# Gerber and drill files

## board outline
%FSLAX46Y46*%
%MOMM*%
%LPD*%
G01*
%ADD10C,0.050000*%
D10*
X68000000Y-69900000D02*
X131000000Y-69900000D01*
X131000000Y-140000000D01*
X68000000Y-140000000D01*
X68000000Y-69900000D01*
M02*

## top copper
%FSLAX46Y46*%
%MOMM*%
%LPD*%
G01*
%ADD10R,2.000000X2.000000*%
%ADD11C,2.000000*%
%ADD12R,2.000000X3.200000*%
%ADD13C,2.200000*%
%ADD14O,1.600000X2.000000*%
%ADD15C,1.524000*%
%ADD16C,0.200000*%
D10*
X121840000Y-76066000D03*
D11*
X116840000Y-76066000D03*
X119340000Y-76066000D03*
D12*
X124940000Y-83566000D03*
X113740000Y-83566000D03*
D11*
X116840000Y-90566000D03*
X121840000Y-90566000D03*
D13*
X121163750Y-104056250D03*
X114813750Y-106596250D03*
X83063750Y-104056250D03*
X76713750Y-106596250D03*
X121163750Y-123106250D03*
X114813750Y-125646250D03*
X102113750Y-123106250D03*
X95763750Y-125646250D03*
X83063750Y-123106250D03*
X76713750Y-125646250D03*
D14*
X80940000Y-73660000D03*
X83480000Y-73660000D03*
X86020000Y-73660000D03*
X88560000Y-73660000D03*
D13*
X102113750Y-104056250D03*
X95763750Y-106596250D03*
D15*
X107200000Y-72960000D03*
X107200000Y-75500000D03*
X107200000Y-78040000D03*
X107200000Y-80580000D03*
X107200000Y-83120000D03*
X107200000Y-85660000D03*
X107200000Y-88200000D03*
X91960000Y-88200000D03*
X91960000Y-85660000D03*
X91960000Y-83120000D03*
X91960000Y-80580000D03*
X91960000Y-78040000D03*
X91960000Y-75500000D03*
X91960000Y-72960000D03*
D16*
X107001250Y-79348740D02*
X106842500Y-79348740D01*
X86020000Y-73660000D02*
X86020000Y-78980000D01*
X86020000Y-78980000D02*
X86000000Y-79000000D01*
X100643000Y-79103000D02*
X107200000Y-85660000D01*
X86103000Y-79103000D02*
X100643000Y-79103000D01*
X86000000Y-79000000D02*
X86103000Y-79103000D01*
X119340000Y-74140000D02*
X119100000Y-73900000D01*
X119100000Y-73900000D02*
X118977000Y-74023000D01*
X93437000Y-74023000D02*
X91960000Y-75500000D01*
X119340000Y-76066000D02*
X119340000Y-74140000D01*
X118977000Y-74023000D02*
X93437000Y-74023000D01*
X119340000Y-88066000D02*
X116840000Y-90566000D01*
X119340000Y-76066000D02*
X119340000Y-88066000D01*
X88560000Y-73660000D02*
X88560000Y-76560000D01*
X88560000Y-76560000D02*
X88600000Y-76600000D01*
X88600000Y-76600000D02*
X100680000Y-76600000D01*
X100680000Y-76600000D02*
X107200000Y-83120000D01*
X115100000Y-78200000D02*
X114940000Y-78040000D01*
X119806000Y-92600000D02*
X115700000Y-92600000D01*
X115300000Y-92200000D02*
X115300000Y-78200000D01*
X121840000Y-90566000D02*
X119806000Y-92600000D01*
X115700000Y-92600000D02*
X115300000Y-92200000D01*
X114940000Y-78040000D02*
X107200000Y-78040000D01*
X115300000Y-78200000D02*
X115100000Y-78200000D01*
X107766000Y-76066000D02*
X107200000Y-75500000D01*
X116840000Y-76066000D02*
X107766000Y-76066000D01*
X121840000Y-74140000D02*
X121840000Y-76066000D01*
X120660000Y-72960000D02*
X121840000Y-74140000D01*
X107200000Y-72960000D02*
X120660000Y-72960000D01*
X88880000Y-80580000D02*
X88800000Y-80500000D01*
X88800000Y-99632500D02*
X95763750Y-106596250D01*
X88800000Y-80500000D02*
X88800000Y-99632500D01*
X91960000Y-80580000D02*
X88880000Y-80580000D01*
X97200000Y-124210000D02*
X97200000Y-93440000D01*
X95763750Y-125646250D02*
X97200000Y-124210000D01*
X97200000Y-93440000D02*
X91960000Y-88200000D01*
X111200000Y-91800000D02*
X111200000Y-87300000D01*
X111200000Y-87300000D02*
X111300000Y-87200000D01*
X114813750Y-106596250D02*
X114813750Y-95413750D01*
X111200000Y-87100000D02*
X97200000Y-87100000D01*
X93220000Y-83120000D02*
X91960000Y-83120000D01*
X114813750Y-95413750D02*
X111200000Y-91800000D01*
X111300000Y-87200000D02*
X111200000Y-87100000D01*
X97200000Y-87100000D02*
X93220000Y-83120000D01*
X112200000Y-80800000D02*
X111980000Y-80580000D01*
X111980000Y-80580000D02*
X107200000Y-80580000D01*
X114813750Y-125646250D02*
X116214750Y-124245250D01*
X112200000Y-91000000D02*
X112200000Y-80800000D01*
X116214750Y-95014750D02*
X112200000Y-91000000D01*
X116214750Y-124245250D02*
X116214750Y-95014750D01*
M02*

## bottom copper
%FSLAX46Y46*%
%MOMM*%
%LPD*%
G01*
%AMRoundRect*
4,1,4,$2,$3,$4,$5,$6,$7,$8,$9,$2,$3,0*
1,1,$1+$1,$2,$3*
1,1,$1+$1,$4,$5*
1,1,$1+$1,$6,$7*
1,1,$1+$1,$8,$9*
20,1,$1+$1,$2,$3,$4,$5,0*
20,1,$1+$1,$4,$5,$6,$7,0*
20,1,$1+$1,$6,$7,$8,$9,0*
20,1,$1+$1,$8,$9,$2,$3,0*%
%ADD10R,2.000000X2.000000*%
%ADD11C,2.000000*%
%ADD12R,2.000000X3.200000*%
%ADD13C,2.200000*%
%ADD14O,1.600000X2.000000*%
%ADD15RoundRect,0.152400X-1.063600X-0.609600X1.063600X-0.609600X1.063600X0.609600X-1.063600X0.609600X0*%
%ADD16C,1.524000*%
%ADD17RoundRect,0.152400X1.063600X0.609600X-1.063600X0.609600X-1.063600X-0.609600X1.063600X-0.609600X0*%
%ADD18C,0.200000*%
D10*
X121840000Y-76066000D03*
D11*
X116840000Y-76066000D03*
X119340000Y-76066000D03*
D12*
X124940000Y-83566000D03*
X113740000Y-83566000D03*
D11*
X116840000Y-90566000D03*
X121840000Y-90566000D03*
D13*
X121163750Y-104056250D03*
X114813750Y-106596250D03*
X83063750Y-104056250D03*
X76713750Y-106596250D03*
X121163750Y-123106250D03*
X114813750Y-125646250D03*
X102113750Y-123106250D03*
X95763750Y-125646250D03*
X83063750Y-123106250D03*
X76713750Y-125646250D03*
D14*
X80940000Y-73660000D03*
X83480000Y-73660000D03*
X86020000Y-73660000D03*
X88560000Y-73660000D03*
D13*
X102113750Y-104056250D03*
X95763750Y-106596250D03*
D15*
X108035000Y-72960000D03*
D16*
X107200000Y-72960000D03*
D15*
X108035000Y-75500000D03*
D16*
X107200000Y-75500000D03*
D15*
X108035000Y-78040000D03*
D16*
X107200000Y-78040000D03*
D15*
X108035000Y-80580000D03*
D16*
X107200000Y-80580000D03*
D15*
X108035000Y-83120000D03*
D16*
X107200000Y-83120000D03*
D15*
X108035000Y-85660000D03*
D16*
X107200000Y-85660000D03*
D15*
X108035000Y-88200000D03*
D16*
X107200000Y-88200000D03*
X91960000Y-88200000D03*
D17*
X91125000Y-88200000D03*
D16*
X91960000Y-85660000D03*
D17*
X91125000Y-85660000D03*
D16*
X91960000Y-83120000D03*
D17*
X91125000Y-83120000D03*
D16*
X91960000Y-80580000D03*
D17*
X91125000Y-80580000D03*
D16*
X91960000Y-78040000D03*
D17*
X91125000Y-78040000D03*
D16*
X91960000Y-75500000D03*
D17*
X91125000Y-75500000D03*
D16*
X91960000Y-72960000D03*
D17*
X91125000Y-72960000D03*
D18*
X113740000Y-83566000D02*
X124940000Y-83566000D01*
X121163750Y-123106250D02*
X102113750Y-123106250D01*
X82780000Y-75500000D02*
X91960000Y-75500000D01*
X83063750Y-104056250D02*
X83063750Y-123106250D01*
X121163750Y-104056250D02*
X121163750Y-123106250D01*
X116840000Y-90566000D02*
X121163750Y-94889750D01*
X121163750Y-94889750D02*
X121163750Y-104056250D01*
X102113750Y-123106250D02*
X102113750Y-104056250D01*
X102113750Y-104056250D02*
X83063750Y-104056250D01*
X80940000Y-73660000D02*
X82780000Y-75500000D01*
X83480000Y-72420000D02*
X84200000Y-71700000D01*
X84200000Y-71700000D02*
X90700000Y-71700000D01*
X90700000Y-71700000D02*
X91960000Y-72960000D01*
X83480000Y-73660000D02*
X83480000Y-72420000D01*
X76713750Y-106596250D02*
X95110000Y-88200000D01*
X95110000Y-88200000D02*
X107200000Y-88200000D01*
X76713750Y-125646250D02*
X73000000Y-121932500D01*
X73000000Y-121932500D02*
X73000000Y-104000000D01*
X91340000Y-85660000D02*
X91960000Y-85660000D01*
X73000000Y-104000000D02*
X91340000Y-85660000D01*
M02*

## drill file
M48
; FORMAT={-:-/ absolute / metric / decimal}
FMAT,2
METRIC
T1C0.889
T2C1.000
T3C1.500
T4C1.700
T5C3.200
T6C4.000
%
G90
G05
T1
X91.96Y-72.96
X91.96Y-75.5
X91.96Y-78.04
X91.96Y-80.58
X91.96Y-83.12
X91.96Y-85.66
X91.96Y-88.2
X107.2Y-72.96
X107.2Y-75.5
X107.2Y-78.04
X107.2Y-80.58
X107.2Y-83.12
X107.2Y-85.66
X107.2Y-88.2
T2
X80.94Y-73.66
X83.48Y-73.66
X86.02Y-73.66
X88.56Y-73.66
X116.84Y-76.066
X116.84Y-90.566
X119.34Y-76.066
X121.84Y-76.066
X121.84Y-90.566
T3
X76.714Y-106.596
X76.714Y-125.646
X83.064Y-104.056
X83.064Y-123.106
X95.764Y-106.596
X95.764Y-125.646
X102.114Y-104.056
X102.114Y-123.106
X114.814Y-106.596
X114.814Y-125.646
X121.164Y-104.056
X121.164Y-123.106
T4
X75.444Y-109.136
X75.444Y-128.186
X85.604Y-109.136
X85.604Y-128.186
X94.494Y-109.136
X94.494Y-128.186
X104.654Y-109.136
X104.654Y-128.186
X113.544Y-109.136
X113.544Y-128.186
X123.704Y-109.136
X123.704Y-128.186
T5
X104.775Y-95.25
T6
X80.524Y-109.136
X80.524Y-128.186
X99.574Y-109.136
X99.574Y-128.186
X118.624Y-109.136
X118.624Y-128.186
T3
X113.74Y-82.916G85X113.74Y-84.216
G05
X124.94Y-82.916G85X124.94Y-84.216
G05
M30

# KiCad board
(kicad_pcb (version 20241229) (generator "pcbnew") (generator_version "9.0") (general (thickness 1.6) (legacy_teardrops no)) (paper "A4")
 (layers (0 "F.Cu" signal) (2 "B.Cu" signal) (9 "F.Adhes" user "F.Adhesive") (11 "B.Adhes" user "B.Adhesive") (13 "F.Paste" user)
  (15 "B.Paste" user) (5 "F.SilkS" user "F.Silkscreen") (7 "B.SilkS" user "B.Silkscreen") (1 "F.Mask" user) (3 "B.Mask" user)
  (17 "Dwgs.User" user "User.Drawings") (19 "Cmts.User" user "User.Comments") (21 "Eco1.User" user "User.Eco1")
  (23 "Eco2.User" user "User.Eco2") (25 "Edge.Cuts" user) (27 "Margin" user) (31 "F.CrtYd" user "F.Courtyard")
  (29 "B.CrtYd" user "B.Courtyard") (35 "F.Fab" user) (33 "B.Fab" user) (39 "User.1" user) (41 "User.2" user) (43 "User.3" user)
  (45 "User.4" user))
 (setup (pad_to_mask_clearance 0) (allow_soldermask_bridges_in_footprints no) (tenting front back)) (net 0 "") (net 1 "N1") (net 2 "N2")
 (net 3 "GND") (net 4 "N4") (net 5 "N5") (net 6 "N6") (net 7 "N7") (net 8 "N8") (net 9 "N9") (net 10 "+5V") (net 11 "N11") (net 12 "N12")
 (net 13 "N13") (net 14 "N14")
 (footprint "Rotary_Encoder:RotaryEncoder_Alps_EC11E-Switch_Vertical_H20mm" (layer "F.Cu") (at 121.84 76.066 -90)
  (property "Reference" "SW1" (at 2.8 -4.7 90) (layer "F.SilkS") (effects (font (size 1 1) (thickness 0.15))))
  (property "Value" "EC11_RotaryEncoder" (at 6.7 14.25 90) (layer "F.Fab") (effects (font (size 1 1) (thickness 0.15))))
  (pad "A" thru_hole rect (at 0 0 270) (size 2 2) (drill 1) (layers "*.Cu" "*.Mask") (remove_unused_layers no) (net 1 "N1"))
  (pad "B" thru_hole circle (at 0 5 270) (size 2 2) (drill 1) (layers "*.Cu" "*.Mask") (remove_unused_layers no) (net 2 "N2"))
  (pad "C" thru_hole circle (at 0 2.5 270) (size 2 2) (drill 1) (layers "*.Cu" "*.Mask") (remove_unused_layers no) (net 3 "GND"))
  (pad "MP" thru_hole rect (at 7.5 -3.1 270) (size 3.2 2) (drill oval 2.8 1.5) (layers "*.Cu" "*.Mask") (remove_unused_layers no))
  (pad "MP" thru_hole rect (at 7.5 8.1 270) (size 3.2 2) (drill oval 2.8 1.5) (layers "*.Cu" "*.Mask") (remove_unused_layers no))
  (pad "S1" thru_hole circle (at 14.5 5 270) (size 2 2) (drill 1) (layers "*.Cu" "*.Mask") (remove_unused_layers no) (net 3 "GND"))
  (pad "S2" thru_hole circle (at 14.5 0 270) (size 2 2) (drill 1) (layers "*.Cu" "*.Mask") (remove_unused_layers no) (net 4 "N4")))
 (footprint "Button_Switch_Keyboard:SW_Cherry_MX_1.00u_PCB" (layer "F.Cu") (at 121.16375 104.05625)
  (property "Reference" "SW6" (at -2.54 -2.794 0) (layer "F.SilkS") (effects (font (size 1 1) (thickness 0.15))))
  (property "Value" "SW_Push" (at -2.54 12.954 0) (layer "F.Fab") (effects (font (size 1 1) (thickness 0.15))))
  (pad "" np_thru_hole circle (at -7.62 5.08) (size 1.7 1.7) (drill 1.7) (layers "*.Cu" "*.Mask"))
  (pad "" np_thru_hole circle (at -2.54 5.08) (size 4 4) (drill 4) (layers "*.Cu" "*.Mask"))
  (pad "" np_thru_hole circle (at 2.54 5.08) (size 1.7 1.7) (drill 1.7) (layers "*.Cu" "*.Mask"))
  (pad "1" thru_hole circle (at 0 0) (size 2.2 2.2) (drill 1.5) (layers "*.Cu" "*.Mask") (remove_unused_layers no) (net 3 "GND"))
  (pad "2" thru_hole circle (at -6.35 2.54) (size 2.2 2.2) (drill 1.5) (layers "*.Cu" "*.Mask") (remove_unused_layers no) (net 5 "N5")))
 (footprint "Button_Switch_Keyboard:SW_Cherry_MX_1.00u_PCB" (layer "F.Cu") (at 83.06375 104.05625)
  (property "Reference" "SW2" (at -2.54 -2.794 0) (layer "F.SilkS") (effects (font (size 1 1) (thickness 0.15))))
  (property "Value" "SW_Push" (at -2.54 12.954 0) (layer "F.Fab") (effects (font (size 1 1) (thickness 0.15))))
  (pad "" np_thru_hole circle (at -7.62 5.08) (size 1.7 1.7) (drill 1.7) (layers "*.Cu" "*.Mask"))
  (pad "" np_thru_hole circle (at -2.54 5.08) (size 4 4) (drill 4) (layers "*.Cu" "*.Mask"))
  (pad "" np_thru_hole circle (at 2.54 5.08) (size 1.7 1.7) (drill 1.7) (layers "*.Cu" "*.Mask"))
  (pad "1" thru_hole circle (at 0 0) (size 2.2 2.2) (drill 1.5) (layers "*.Cu" "*.Mask") (remove_unused_layers no) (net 3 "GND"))
  (pad "2" thru_hole circle (at -6.35 2.54) (size 2.2 2.2) (drill 1.5) (layers "*.Cu" "*.Mask") (remove_unused_layers no) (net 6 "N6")))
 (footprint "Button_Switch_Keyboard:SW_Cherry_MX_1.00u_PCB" (layer "F.Cu") (at 121.16375 123.10625)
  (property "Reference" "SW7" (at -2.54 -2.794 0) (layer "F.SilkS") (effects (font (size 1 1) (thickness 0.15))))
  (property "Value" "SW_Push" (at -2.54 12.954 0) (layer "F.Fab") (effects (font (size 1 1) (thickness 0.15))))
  (pad "" np_thru_hole circle (at -7.62 5.08) (size 1.7 1.7) (drill 1.7) (layers "*.Cu" "*.Mask"))
  (pad "" np_thru_hole circle (at -2.54 5.08) (size 4 4) (drill 4) (layers "*.Cu" "*.Mask"))
  (pad "" np_thru_hole circle (at 2.54 5.08) (size 1.7 1.7) (drill 1.7) (layers "*.Cu" "*.Mask"))
  (pad "1" thru_hole circle (at 0 0) (size 2.2 2.2) (drill 1.5) (layers "*.Cu" "*.Mask") (remove_unused_layers no) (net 3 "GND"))
  (pad "2" thru_hole circle (at -6.35 2.54) (size 2.2 2.2) (drill 1.5) (layers "*.Cu" "*.Mask") (remove_unused_layers no) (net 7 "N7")))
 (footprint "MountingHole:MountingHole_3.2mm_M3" (layer "F.Cu") (at 104.775 95.25)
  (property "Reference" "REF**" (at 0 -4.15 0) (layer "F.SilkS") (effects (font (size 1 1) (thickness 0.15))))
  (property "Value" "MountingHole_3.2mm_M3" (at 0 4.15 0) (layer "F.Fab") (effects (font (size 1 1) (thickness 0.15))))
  (pad "" np_thru_hole circle (at 0 0) (size 3.2 3.2) (drill 3.2) (layers "*.Cu" "*.Mask")))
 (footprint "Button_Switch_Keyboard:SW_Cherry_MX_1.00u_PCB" (layer "F.Cu") (at 102.11375 123.10625)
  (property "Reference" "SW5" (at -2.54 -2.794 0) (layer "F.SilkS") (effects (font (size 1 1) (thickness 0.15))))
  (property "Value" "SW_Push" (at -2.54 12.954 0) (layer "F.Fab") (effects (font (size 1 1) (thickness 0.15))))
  (pad "" np_thru_hole circle (at -7.62 5.08) (size 1.7 1.7) (drill 1.7) (layers "*.Cu" "*.Mask"))
  (pad "" np_thru_hole circle (at -2.54 5.08) (size 4 4) (drill 4) (layers "*.Cu" "*.Mask"))
  (pad "" np_thru_hole circle (at 2.54 5.08) (size 1.7 1.7) (drill 1.7) (layers "*.Cu" "*.Mask"))
  (pad "1" thru_hole circle (at 0 0) (size 2.2 2.2) (drill 1.5) (layers "*.Cu" "*.Mask") (remove_unused_layers no) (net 3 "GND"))
  (pad "2" thru_hole circle (at -6.35 2.54) (size 2.2 2.2) (drill 1.5) (layers "*.Cu" "*.Mask") (remove_unused_layers no) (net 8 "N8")))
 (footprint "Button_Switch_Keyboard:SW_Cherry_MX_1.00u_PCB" (layer "F.Cu") (at 83.06375 123.10625)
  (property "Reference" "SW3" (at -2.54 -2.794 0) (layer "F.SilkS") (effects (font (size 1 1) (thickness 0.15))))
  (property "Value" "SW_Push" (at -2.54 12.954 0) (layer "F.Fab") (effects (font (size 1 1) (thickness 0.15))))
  (pad "" np_thru_hole circle (at -7.62 5.08) (size 1.7 1.7) (drill 1.7) (layers "*.Cu" "*.Mask"))
  (pad "" np_thru_hole circle (at -2.54 5.08) (size 4 4) (drill 4) (layers "*.Cu" "*.Mask"))
  (pad "" np_thru_hole circle (at 2.54 5.08) (size 1.7 1.7) (drill 1.7) (layers "*.Cu" "*.Mask"))
  (pad "1" thru_hole circle (at 0 0) (size 2.2 2.2) (drill 1.5) (layers "*.Cu" "*.Mask") (remove_unused_layers no) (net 3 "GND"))
  (pad "2" thru_hole circle (at -6.35 2.54) (size 2.2 2.2) (drill 1.5) (layers "*.Cu" "*.Mask") (remove_unused_layers no) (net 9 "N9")))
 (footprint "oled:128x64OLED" (layer "F.Cu") (at 84.56 84.26)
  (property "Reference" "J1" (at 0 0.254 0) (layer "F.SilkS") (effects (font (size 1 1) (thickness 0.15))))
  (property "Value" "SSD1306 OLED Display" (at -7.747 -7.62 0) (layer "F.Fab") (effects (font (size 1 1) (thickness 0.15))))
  (pad "1" thru_hole oval (at -3.62 -10.6 90) (size 2 1.6) (drill 1) (layers "*.Cu" "*.Mask") (remove_unused_layers no) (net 3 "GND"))
  (pad "2" thru_hole oval (at -1.08 -10.6 90) (size 2 1.6) (drill 1) (layers "*.Cu" "*.Mask") (remove_unused_layers no) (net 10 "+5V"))
  (pad "3" thru_hole oval (at 1.46 -10.6 90) (size 2 1.6) (drill 1) (layers "*.Cu" "*.Mask") (remove_unused_layers no) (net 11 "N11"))
  (pad "4" thru_hole oval (at 4 -10.6 90) (size 2 1.6) (drill 1) (layers "*.Cu" "*.Mask") (remove_unused_layers no) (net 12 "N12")))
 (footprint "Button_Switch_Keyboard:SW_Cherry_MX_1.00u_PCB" (layer "F.Cu") (at 102.11375 104.05625)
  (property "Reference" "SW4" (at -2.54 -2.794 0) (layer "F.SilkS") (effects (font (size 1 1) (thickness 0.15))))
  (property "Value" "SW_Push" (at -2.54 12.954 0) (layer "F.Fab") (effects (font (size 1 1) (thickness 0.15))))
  (pad "" np_thru_hole circle (at -7.62 5.08) (size 1.7 1.7) (drill 1.7) (layers "*.Cu" "*.Mask"))
  (pad "" np_thru_hole circle (at -2.54 5.08) (size 4 4) (drill 4) (layers "*.Cu" "*.Mask"))
  (pad "" np_thru_hole circle (at 2.54 5.08) (size 1.7 1.7) (drill 1.7) (layers "*.Cu" "*.Mask"))
  (pad "1" thru_hole circle (at 0 0) (size 2.2 2.2) (drill 1.5) (layers "*.Cu" "*.Mask") (remove_unused_layers no) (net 3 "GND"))
  (pad "2" thru_hole circle (at -6.35 2.54) (size 2.2 2.2) (drill 1.5) (layers "*.Cu" "*.Mask") (remove_unused_layers no) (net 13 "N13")))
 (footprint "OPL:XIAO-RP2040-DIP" (layer "B.Cu") (at 99.58 80.58 180)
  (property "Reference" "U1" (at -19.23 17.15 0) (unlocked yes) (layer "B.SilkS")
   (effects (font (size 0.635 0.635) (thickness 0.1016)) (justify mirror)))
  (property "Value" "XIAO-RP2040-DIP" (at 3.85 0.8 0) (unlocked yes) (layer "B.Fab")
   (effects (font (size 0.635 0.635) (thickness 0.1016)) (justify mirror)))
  (pad "1" smd roundrect (at -8.455 7.62) (size 2.432 1.524) (layers "B.Cu" "B.Mask") (roundrect_rratio 0.1) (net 1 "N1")
   (thermal_bridge_angle 45))
  (pad "1" thru_hole circle (at -7.62 7.62) (size 1.524 1.524) (drill 0.889) (layers "*.Cu" "*.Mask") (remove_unused_layers no) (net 1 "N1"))
  (pad "2" smd roundrect (at -8.455 5.08) (size 2.432 1.524) (layers "B.Cu" "B.Mask") (roundrect_rratio 0.1) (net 2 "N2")
   (thermal_bridge_angle 45))
  (pad "2" thru_hole circle (at -7.62 5.08) (size 1.524 1.524) (drill 0.889) (layers "*.Cu" "*.Mask") (remove_unused_layers no) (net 2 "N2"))
  (pad "3" smd roundrect (at -8.455 2.54) (size 2.432 1.524) (layers "B.Cu" "B.Mask") (roundrect_rratio 0.1) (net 4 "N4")
   (thermal_bridge_angle 45))
  (pad "3" thru_hole circle (at -7.62 2.54) (size 1.524 1.524) (drill 0.889) (layers "*.Cu" "*.Mask") (remove_unused_layers no) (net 4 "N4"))
  (pad "4" smd roundrect (at -8.455 0) (size 2.432 1.524) (layers "B.Cu" "B.Mask") (roundrect_rratio 0.1) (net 7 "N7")
   (thermal_bridge_angle 45))
  (pad "4" thru_hole circle (at -7.62 0) (size 1.524 1.524) (drill 0.889) (layers "*.Cu" "*.Mask") (remove_unused_layers no) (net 7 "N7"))
  (pad "5" smd roundrect (at -8.455 -2.54) (size 2.432 1.524) (layers "B.Cu" "B.Mask") (roundrect_rratio 0.1) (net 12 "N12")
   (thermal_bridge_angle 45))
  (pad "5" thru_hole circle (at -7.62 -2.54) (size 1.524 1.524) (drill 0.889) (layers "*.Cu" "*.Mask") (remove_unused_layers no)
   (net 12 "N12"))
  (pad "6" smd roundrect (at -8.455 -5.08) (size 2.432 1.524) (layers "B.Cu" "B.Mask") (roundrect_rratio 0.1) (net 11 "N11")
   (thermal_bridge_angle 45))
  (pad "6" thru_hole circle (at -7.62 -5.08) (size 1.524 1.524) (drill 0.889) (layers "*.Cu" "*.Mask") (remove_unused_layers no)
   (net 11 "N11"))
  (pad "7" smd roundrect (at -8.455 -7.62) (size 2.432 1.524) (layers "B.Cu" "B.Mask") (roundrect_rratio 0.1) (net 6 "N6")
   (thermal_bridge_angle 45))
  (pad "7" thru_hole circle (at -7.62 -7.62) (size 1.524 1.524) (drill 0.889) (layers "*.Cu" "*.Mask") (remove_unused_layers no)
   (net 6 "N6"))
  (pad "8" thru_hole circle (at 7.62 -7.62 180) (size 1.524 1.524) (drill 0.889) (layers "*.Cu" "*.Mask") (remove_unused_layers no)
   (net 8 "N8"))
  (pad "8" smd roundrect (at 8.455 -7.62 180) (size 2.432 1.524) (layers "B.Cu" "B.Mask") (roundrect_rratio 0.1) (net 8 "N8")
   (thermal_bridge_angle 45))
  (pad "9" thru_hole circle (at 7.62 -5.08 180) (size 1.524 1.524) (drill 0.889) (layers "*.Cu" "*.Mask") (remove_unused_layers no)
   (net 9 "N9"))
  (pad "9" smd roundrect (at 8.455 -5.08 180) (size 2.432 1.524) (layers "B.Cu" "B.Mask") (roundrect_rratio 0.1) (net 9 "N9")
   (thermal_bridge_angle 45))
  (pad "10" thru_hole circle (at 7.62 -2.54 180) (size 1.524 1.524) (drill 0.889) (layers "*.Cu" "*.Mask") (remove_unused_layers no)
   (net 5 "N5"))
  (pad "10" smd roundrect (at 8.455 -2.54 180) (size 2.432 1.524) (layers "B.Cu" "B.Mask") (roundrect_rratio 0.1) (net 5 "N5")
   (thermal_bridge_angle 45))
  (pad "11" thru_hole circle (at 7.62 0 180) (size 1.524 1.524) (drill 0.889) (layers "*.Cu" "*.Mask") (remove_unused_layers no)
   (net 13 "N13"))
  (pad "11" smd roundrect (at 8.455 0 180) (size 2.432 1.524) (layers "B.Cu" "B.Mask") (roundrect_rratio 0.1) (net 13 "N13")
   (thermal_bridge_angle 45))
  (pad "12" thru_hole circle (at 7.62 2.54 180) (size 1.524 1.524) (drill 0.889) (layers "*.Cu" "*.Mask") (remove_unused_layers no)
   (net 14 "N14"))
  (pad "12" smd roundrect (at 8.455 2.54 180) (size 2.432 1.524) (layers "B.Cu" "B.Mask") (roundrect_rratio 0.1) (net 14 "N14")
   (thermal_bridge_angle 45))
  (pad "13" thru_hole circle (at 7.62 5.08 180) (size 1.524 1.524) (drill 0.889) (layers "*.Cu" "*.Mask") (remove_unused_layers no)
   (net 3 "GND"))
  (pad "13" smd roundrect (at 8.455 5.08 180) (size 2.432 1.524) (layers "B.Cu" "B.Mask") (roundrect_rratio 0.1) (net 3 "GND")
   (thermal_bridge_angle 45))
  (pad "14" thru_hole circle (at 7.62 7.62 180) (size 1.524 1.524) (drill 0.889) (layers "*.Cu" "*.Mask") (remove_unused_layers no)
   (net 10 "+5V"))
  (pad "14" smd roundrect (at 8.455 7.62 180) (size 2.432 1.524) (layers "B.Cu" "B.Mask") (roundrect_rratio 0.1) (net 10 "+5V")
   (thermal_bridge_angle 45)))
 (gr_rect (start 68 69.9) (end 131 140) (stroke (width 0.05) (type default)) (fill no) (layer "Edge.Cuts"))
 (segment (start 107.00125 79.34874) (end 106.8425 79.34874) (width 0.2) (layer "F.Cu") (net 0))
 (segment (start 113.74 83.566) (end 124.94 83.566) (width 0.2) (layer "B.Cu") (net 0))
 (segment (start 86.02 73.66) (end 86.02 78.98) (width 0.2) (layer "F.Cu") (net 11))
 (segment (start 86.02 78.98) (end 86 79) (width 0.2) (layer "F.Cu") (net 11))
 (segment (start 100.643 79.103) (end 107.2 85.66) (width 0.2) (layer "F.Cu") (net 11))
 (segment (start 86.103 79.103) (end 100.643 79.103) (width 0.2) (layer "F.Cu") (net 11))
 (segment (start 86 79) (end 86.103 79.103) (width 0.2) (layer "F.Cu") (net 11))
 (segment (start 119.34 74.14) (end 119.1 73.9) (width 0.2) (layer "F.Cu") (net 3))
 (segment (start 119.1 73.9) (end 118.977 74.023) (width 0.2) (layer "F.Cu") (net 3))
 (segment (start 93.437 74.023) (end 91.96 75.5) (width 0.2) (layer "F.Cu") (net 3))
 (segment (start 119.34 76.066) (end 119.34 74.14) (width 0.2) (layer "F.Cu") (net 3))
 (segment (start 118.977 74.023) (end 93.437 74.023) (width 0.2) (layer "F.Cu") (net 3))
 (segment (start 119.34 88.066) (end 116.84 90.566) (width 0.2) (layer "F.Cu") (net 3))
 (segment (start 119.34 76.066) (end 119.34 88.066) (width 0.2) (layer "F.Cu") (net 3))
 (segment (start 121.16375 123.10625) (end 102.11375 123.10625) (width 0.2) (layer "B.Cu") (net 3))
 (segment (start 82.78 75.5) (end 91.96 75.5) (width 0.2) (layer "B.Cu") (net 3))
 (segment (start 83.06375 104.05625) (end 83.06375 123.10625) (width 0.2) (layer "B.Cu") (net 3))
 (segment (start 121.16375 104.05625) (end 121.16375 123.10625) (width 0.2) (layer "B.Cu") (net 3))
 (segment (start 116.84 90.566) (end 121.16375 94.88975) (width 0.2) (layer "B.Cu") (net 3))
 (segment (start 121.16375 94.88975) (end 121.16375 104.05625) (width 0.2) (layer "B.Cu") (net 3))
 (segment (start 102.11375 123.10625) (end 102.11375 104.05625) (width 0.2) (layer "B.Cu") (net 3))
 (segment (start 102.11375 104.05625) (end 83.06375 104.05625) (width 0.2) (layer "B.Cu") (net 3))
 (segment (start 80.94 73.66) (end 82.78 75.5) (width 0.2) (layer "B.Cu") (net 3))
 (segment (start 88.56 73.66) (end 88.56 76.56) (width 0.2) (layer "F.Cu") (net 12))
 (segment (start 88.56 76.56) (end 88.6 76.6) (width 0.2) (layer "F.Cu") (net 12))
 (segment (start 88.6 76.6) (end 100.68 76.6) (width 0.2) (layer "F.Cu") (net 12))
 (segment (start 100.68 76.6) (end 107.2 83.12) (width 0.2) (layer "F.Cu") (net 12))
 (segment (start 83.48 72.42) (end 84.2 71.7) (width 0.2) (layer "B.Cu") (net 10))
 (segment (start 84.2 71.7) (end 90.7 71.7) (width 0.2) (layer "B.Cu") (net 10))
 (segment (start 90.7 71.7) (end 91.96 72.96) (width 0.2) (layer "B.Cu") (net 10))
 (segment (start 83.48 73.66) (end 83.48 72.42) (width 0.2) (layer "B.Cu") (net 10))
 (segment (start 115.1 78.2) (end 114.94 78.04) (width 0.2) (layer "F.Cu") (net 4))
 (segment (start 119.806 92.6) (end 115.7 92.6) (width 0.2) (layer "F.Cu") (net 4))
 (segment (start 115.3 92.2) (end 115.3 78.2) (width 0.2) (layer "F.Cu") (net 4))
 (segment (start 121.84 90.566) (end 119.806 92.6) (width 0.2) (layer "F.Cu") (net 4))
 (segment (start 115.7 92.6) (end 115.3 92.2) (width 0.2) (layer "F.Cu") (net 4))
 (segment (start 114.94 78.04) (end 107.2 78.04) (width 0.2) (layer "F.Cu") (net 4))
 (segment (start 115.3 78.2) (end 115.1 78.2) (width 0.2) (layer "F.Cu") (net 4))
 (segment (start 107.766 76.066) (end 107.2 75.5) (width 0.2) (layer "F.Cu") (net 2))
 (segment (start 116.84 76.066) (end 107.766 76.066) (width 0.2) (layer "F.Cu") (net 2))
 (segment (start 121.84 74.14) (end 121.84 76.066) (width 0.2) (layer "F.Cu") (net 1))
 (segment (start 120.66 72.96) (end 121.84 74.14) (width 0.2) (layer "F.Cu") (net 1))
 (segment (start 107.2 72.96) (end 120.66 72.96) (width 0.2) (layer "F.Cu") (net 1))
 (segment (start 76.71375 106.59625) (end 95.11 88.2) (width 0.2) (layer "B.Cu") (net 6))
 (segment (start 95.11 88.2) (end 107.2 88.2) (width 0.2) (layer "B.Cu") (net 6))
 (segment (start 76.71375 125.64625) (end 73 121.9325) (width 0.2) (layer "B.Cu") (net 9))
 (segment (start 73 121.9325) (end 73 104) (width 0.2) (layer "B.Cu") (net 9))
 (segment (start 91.34 85.66) (end 91.96 85.66) (width 0.2) (layer "B.Cu") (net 9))
 (segment (start 73 104) (end 91.34 85.66) (width 0.2) (layer "B.Cu") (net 9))
 (segment (start 88.88 80.58) (end 88.8 80.5) (width 0.2) (layer "F.Cu") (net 13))
 (segment (start 88.8 99.6325) (end 95.76375 106.59625) (width 0.2) (layer "F.Cu") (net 13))
 (segment (start 88.8 80.5) (end 88.8 99.6325) (width 0.2) (layer "F.Cu") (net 13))
 (segment (start 91.96 80.58) (end 88.88 80.58) (width 0.2) (layer "F.Cu") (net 13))
 (segment (start 97.2 124.21) (end 97.2 93.44) (width 0.2) (layer "F.Cu") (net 8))
 (segment (start 95.76375 125.64625) (end 97.2 124.21) (width 0.2) (layer "F.Cu") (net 8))
 (segment (start 97.2 93.44) (end 91.96 88.2) (width 0.2) (layer "F.Cu") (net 8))
 (segment (start 111.2 91.8) (end 111.2 87.3) (width 0.2) (layer "F.Cu") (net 5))
 (segment (start 111.2 87.3) (end 111.3 87.2) (width 0.2) (layer "F.Cu") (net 5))
 (segment (start 114.81375 106.59625) (end 114.81375 95.41375) (width 0.2) (layer "F.Cu") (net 5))
 (segment (start 111.2 87.1) (end 97.2 87.1) (width 0.2) (layer "F.Cu") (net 5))
 (segment (start 93.22 83.12) (end 91.96 83.12) (width 0.2) (layer "F.Cu") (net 5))
 (segment (start 114.81375 95.41375) (end 111.2 91.8) (width 0.2) (layer "F.Cu") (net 5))
 (segment (start 111.3 87.2) (end 111.2 87.1) (width 0.2) (layer "F.Cu") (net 5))
 (segment (start 97.2 87.1) (end 93.22 83.12) (width 0.2) (layer "F.Cu") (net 5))
 (segment (start 112.2 80.8) (end 111.98 80.58) (width 0.2) (layer "F.Cu") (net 7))
 (segment (start 111.98 80.58) (end 107.2 80.58) (width 0.2) (layer "F.Cu") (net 7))
 (segment (start 114.81375 125.64625) (end 116.21475 124.24525) (width 0.2) (layer "F.Cu") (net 7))
 (segment (start 112.2 91) (end 112.2 80.8) (width 0.2) (layer "F.Cu") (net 7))
 (segment (start 116.21475 95.01475) (end 112.2 91) (width 0.2) (layer "F.Cu") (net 7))
 (segment (start 116.21475 124.24525) (end 116.21475 95.01475) (width 0.2) (layer "F.Cu") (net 7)))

